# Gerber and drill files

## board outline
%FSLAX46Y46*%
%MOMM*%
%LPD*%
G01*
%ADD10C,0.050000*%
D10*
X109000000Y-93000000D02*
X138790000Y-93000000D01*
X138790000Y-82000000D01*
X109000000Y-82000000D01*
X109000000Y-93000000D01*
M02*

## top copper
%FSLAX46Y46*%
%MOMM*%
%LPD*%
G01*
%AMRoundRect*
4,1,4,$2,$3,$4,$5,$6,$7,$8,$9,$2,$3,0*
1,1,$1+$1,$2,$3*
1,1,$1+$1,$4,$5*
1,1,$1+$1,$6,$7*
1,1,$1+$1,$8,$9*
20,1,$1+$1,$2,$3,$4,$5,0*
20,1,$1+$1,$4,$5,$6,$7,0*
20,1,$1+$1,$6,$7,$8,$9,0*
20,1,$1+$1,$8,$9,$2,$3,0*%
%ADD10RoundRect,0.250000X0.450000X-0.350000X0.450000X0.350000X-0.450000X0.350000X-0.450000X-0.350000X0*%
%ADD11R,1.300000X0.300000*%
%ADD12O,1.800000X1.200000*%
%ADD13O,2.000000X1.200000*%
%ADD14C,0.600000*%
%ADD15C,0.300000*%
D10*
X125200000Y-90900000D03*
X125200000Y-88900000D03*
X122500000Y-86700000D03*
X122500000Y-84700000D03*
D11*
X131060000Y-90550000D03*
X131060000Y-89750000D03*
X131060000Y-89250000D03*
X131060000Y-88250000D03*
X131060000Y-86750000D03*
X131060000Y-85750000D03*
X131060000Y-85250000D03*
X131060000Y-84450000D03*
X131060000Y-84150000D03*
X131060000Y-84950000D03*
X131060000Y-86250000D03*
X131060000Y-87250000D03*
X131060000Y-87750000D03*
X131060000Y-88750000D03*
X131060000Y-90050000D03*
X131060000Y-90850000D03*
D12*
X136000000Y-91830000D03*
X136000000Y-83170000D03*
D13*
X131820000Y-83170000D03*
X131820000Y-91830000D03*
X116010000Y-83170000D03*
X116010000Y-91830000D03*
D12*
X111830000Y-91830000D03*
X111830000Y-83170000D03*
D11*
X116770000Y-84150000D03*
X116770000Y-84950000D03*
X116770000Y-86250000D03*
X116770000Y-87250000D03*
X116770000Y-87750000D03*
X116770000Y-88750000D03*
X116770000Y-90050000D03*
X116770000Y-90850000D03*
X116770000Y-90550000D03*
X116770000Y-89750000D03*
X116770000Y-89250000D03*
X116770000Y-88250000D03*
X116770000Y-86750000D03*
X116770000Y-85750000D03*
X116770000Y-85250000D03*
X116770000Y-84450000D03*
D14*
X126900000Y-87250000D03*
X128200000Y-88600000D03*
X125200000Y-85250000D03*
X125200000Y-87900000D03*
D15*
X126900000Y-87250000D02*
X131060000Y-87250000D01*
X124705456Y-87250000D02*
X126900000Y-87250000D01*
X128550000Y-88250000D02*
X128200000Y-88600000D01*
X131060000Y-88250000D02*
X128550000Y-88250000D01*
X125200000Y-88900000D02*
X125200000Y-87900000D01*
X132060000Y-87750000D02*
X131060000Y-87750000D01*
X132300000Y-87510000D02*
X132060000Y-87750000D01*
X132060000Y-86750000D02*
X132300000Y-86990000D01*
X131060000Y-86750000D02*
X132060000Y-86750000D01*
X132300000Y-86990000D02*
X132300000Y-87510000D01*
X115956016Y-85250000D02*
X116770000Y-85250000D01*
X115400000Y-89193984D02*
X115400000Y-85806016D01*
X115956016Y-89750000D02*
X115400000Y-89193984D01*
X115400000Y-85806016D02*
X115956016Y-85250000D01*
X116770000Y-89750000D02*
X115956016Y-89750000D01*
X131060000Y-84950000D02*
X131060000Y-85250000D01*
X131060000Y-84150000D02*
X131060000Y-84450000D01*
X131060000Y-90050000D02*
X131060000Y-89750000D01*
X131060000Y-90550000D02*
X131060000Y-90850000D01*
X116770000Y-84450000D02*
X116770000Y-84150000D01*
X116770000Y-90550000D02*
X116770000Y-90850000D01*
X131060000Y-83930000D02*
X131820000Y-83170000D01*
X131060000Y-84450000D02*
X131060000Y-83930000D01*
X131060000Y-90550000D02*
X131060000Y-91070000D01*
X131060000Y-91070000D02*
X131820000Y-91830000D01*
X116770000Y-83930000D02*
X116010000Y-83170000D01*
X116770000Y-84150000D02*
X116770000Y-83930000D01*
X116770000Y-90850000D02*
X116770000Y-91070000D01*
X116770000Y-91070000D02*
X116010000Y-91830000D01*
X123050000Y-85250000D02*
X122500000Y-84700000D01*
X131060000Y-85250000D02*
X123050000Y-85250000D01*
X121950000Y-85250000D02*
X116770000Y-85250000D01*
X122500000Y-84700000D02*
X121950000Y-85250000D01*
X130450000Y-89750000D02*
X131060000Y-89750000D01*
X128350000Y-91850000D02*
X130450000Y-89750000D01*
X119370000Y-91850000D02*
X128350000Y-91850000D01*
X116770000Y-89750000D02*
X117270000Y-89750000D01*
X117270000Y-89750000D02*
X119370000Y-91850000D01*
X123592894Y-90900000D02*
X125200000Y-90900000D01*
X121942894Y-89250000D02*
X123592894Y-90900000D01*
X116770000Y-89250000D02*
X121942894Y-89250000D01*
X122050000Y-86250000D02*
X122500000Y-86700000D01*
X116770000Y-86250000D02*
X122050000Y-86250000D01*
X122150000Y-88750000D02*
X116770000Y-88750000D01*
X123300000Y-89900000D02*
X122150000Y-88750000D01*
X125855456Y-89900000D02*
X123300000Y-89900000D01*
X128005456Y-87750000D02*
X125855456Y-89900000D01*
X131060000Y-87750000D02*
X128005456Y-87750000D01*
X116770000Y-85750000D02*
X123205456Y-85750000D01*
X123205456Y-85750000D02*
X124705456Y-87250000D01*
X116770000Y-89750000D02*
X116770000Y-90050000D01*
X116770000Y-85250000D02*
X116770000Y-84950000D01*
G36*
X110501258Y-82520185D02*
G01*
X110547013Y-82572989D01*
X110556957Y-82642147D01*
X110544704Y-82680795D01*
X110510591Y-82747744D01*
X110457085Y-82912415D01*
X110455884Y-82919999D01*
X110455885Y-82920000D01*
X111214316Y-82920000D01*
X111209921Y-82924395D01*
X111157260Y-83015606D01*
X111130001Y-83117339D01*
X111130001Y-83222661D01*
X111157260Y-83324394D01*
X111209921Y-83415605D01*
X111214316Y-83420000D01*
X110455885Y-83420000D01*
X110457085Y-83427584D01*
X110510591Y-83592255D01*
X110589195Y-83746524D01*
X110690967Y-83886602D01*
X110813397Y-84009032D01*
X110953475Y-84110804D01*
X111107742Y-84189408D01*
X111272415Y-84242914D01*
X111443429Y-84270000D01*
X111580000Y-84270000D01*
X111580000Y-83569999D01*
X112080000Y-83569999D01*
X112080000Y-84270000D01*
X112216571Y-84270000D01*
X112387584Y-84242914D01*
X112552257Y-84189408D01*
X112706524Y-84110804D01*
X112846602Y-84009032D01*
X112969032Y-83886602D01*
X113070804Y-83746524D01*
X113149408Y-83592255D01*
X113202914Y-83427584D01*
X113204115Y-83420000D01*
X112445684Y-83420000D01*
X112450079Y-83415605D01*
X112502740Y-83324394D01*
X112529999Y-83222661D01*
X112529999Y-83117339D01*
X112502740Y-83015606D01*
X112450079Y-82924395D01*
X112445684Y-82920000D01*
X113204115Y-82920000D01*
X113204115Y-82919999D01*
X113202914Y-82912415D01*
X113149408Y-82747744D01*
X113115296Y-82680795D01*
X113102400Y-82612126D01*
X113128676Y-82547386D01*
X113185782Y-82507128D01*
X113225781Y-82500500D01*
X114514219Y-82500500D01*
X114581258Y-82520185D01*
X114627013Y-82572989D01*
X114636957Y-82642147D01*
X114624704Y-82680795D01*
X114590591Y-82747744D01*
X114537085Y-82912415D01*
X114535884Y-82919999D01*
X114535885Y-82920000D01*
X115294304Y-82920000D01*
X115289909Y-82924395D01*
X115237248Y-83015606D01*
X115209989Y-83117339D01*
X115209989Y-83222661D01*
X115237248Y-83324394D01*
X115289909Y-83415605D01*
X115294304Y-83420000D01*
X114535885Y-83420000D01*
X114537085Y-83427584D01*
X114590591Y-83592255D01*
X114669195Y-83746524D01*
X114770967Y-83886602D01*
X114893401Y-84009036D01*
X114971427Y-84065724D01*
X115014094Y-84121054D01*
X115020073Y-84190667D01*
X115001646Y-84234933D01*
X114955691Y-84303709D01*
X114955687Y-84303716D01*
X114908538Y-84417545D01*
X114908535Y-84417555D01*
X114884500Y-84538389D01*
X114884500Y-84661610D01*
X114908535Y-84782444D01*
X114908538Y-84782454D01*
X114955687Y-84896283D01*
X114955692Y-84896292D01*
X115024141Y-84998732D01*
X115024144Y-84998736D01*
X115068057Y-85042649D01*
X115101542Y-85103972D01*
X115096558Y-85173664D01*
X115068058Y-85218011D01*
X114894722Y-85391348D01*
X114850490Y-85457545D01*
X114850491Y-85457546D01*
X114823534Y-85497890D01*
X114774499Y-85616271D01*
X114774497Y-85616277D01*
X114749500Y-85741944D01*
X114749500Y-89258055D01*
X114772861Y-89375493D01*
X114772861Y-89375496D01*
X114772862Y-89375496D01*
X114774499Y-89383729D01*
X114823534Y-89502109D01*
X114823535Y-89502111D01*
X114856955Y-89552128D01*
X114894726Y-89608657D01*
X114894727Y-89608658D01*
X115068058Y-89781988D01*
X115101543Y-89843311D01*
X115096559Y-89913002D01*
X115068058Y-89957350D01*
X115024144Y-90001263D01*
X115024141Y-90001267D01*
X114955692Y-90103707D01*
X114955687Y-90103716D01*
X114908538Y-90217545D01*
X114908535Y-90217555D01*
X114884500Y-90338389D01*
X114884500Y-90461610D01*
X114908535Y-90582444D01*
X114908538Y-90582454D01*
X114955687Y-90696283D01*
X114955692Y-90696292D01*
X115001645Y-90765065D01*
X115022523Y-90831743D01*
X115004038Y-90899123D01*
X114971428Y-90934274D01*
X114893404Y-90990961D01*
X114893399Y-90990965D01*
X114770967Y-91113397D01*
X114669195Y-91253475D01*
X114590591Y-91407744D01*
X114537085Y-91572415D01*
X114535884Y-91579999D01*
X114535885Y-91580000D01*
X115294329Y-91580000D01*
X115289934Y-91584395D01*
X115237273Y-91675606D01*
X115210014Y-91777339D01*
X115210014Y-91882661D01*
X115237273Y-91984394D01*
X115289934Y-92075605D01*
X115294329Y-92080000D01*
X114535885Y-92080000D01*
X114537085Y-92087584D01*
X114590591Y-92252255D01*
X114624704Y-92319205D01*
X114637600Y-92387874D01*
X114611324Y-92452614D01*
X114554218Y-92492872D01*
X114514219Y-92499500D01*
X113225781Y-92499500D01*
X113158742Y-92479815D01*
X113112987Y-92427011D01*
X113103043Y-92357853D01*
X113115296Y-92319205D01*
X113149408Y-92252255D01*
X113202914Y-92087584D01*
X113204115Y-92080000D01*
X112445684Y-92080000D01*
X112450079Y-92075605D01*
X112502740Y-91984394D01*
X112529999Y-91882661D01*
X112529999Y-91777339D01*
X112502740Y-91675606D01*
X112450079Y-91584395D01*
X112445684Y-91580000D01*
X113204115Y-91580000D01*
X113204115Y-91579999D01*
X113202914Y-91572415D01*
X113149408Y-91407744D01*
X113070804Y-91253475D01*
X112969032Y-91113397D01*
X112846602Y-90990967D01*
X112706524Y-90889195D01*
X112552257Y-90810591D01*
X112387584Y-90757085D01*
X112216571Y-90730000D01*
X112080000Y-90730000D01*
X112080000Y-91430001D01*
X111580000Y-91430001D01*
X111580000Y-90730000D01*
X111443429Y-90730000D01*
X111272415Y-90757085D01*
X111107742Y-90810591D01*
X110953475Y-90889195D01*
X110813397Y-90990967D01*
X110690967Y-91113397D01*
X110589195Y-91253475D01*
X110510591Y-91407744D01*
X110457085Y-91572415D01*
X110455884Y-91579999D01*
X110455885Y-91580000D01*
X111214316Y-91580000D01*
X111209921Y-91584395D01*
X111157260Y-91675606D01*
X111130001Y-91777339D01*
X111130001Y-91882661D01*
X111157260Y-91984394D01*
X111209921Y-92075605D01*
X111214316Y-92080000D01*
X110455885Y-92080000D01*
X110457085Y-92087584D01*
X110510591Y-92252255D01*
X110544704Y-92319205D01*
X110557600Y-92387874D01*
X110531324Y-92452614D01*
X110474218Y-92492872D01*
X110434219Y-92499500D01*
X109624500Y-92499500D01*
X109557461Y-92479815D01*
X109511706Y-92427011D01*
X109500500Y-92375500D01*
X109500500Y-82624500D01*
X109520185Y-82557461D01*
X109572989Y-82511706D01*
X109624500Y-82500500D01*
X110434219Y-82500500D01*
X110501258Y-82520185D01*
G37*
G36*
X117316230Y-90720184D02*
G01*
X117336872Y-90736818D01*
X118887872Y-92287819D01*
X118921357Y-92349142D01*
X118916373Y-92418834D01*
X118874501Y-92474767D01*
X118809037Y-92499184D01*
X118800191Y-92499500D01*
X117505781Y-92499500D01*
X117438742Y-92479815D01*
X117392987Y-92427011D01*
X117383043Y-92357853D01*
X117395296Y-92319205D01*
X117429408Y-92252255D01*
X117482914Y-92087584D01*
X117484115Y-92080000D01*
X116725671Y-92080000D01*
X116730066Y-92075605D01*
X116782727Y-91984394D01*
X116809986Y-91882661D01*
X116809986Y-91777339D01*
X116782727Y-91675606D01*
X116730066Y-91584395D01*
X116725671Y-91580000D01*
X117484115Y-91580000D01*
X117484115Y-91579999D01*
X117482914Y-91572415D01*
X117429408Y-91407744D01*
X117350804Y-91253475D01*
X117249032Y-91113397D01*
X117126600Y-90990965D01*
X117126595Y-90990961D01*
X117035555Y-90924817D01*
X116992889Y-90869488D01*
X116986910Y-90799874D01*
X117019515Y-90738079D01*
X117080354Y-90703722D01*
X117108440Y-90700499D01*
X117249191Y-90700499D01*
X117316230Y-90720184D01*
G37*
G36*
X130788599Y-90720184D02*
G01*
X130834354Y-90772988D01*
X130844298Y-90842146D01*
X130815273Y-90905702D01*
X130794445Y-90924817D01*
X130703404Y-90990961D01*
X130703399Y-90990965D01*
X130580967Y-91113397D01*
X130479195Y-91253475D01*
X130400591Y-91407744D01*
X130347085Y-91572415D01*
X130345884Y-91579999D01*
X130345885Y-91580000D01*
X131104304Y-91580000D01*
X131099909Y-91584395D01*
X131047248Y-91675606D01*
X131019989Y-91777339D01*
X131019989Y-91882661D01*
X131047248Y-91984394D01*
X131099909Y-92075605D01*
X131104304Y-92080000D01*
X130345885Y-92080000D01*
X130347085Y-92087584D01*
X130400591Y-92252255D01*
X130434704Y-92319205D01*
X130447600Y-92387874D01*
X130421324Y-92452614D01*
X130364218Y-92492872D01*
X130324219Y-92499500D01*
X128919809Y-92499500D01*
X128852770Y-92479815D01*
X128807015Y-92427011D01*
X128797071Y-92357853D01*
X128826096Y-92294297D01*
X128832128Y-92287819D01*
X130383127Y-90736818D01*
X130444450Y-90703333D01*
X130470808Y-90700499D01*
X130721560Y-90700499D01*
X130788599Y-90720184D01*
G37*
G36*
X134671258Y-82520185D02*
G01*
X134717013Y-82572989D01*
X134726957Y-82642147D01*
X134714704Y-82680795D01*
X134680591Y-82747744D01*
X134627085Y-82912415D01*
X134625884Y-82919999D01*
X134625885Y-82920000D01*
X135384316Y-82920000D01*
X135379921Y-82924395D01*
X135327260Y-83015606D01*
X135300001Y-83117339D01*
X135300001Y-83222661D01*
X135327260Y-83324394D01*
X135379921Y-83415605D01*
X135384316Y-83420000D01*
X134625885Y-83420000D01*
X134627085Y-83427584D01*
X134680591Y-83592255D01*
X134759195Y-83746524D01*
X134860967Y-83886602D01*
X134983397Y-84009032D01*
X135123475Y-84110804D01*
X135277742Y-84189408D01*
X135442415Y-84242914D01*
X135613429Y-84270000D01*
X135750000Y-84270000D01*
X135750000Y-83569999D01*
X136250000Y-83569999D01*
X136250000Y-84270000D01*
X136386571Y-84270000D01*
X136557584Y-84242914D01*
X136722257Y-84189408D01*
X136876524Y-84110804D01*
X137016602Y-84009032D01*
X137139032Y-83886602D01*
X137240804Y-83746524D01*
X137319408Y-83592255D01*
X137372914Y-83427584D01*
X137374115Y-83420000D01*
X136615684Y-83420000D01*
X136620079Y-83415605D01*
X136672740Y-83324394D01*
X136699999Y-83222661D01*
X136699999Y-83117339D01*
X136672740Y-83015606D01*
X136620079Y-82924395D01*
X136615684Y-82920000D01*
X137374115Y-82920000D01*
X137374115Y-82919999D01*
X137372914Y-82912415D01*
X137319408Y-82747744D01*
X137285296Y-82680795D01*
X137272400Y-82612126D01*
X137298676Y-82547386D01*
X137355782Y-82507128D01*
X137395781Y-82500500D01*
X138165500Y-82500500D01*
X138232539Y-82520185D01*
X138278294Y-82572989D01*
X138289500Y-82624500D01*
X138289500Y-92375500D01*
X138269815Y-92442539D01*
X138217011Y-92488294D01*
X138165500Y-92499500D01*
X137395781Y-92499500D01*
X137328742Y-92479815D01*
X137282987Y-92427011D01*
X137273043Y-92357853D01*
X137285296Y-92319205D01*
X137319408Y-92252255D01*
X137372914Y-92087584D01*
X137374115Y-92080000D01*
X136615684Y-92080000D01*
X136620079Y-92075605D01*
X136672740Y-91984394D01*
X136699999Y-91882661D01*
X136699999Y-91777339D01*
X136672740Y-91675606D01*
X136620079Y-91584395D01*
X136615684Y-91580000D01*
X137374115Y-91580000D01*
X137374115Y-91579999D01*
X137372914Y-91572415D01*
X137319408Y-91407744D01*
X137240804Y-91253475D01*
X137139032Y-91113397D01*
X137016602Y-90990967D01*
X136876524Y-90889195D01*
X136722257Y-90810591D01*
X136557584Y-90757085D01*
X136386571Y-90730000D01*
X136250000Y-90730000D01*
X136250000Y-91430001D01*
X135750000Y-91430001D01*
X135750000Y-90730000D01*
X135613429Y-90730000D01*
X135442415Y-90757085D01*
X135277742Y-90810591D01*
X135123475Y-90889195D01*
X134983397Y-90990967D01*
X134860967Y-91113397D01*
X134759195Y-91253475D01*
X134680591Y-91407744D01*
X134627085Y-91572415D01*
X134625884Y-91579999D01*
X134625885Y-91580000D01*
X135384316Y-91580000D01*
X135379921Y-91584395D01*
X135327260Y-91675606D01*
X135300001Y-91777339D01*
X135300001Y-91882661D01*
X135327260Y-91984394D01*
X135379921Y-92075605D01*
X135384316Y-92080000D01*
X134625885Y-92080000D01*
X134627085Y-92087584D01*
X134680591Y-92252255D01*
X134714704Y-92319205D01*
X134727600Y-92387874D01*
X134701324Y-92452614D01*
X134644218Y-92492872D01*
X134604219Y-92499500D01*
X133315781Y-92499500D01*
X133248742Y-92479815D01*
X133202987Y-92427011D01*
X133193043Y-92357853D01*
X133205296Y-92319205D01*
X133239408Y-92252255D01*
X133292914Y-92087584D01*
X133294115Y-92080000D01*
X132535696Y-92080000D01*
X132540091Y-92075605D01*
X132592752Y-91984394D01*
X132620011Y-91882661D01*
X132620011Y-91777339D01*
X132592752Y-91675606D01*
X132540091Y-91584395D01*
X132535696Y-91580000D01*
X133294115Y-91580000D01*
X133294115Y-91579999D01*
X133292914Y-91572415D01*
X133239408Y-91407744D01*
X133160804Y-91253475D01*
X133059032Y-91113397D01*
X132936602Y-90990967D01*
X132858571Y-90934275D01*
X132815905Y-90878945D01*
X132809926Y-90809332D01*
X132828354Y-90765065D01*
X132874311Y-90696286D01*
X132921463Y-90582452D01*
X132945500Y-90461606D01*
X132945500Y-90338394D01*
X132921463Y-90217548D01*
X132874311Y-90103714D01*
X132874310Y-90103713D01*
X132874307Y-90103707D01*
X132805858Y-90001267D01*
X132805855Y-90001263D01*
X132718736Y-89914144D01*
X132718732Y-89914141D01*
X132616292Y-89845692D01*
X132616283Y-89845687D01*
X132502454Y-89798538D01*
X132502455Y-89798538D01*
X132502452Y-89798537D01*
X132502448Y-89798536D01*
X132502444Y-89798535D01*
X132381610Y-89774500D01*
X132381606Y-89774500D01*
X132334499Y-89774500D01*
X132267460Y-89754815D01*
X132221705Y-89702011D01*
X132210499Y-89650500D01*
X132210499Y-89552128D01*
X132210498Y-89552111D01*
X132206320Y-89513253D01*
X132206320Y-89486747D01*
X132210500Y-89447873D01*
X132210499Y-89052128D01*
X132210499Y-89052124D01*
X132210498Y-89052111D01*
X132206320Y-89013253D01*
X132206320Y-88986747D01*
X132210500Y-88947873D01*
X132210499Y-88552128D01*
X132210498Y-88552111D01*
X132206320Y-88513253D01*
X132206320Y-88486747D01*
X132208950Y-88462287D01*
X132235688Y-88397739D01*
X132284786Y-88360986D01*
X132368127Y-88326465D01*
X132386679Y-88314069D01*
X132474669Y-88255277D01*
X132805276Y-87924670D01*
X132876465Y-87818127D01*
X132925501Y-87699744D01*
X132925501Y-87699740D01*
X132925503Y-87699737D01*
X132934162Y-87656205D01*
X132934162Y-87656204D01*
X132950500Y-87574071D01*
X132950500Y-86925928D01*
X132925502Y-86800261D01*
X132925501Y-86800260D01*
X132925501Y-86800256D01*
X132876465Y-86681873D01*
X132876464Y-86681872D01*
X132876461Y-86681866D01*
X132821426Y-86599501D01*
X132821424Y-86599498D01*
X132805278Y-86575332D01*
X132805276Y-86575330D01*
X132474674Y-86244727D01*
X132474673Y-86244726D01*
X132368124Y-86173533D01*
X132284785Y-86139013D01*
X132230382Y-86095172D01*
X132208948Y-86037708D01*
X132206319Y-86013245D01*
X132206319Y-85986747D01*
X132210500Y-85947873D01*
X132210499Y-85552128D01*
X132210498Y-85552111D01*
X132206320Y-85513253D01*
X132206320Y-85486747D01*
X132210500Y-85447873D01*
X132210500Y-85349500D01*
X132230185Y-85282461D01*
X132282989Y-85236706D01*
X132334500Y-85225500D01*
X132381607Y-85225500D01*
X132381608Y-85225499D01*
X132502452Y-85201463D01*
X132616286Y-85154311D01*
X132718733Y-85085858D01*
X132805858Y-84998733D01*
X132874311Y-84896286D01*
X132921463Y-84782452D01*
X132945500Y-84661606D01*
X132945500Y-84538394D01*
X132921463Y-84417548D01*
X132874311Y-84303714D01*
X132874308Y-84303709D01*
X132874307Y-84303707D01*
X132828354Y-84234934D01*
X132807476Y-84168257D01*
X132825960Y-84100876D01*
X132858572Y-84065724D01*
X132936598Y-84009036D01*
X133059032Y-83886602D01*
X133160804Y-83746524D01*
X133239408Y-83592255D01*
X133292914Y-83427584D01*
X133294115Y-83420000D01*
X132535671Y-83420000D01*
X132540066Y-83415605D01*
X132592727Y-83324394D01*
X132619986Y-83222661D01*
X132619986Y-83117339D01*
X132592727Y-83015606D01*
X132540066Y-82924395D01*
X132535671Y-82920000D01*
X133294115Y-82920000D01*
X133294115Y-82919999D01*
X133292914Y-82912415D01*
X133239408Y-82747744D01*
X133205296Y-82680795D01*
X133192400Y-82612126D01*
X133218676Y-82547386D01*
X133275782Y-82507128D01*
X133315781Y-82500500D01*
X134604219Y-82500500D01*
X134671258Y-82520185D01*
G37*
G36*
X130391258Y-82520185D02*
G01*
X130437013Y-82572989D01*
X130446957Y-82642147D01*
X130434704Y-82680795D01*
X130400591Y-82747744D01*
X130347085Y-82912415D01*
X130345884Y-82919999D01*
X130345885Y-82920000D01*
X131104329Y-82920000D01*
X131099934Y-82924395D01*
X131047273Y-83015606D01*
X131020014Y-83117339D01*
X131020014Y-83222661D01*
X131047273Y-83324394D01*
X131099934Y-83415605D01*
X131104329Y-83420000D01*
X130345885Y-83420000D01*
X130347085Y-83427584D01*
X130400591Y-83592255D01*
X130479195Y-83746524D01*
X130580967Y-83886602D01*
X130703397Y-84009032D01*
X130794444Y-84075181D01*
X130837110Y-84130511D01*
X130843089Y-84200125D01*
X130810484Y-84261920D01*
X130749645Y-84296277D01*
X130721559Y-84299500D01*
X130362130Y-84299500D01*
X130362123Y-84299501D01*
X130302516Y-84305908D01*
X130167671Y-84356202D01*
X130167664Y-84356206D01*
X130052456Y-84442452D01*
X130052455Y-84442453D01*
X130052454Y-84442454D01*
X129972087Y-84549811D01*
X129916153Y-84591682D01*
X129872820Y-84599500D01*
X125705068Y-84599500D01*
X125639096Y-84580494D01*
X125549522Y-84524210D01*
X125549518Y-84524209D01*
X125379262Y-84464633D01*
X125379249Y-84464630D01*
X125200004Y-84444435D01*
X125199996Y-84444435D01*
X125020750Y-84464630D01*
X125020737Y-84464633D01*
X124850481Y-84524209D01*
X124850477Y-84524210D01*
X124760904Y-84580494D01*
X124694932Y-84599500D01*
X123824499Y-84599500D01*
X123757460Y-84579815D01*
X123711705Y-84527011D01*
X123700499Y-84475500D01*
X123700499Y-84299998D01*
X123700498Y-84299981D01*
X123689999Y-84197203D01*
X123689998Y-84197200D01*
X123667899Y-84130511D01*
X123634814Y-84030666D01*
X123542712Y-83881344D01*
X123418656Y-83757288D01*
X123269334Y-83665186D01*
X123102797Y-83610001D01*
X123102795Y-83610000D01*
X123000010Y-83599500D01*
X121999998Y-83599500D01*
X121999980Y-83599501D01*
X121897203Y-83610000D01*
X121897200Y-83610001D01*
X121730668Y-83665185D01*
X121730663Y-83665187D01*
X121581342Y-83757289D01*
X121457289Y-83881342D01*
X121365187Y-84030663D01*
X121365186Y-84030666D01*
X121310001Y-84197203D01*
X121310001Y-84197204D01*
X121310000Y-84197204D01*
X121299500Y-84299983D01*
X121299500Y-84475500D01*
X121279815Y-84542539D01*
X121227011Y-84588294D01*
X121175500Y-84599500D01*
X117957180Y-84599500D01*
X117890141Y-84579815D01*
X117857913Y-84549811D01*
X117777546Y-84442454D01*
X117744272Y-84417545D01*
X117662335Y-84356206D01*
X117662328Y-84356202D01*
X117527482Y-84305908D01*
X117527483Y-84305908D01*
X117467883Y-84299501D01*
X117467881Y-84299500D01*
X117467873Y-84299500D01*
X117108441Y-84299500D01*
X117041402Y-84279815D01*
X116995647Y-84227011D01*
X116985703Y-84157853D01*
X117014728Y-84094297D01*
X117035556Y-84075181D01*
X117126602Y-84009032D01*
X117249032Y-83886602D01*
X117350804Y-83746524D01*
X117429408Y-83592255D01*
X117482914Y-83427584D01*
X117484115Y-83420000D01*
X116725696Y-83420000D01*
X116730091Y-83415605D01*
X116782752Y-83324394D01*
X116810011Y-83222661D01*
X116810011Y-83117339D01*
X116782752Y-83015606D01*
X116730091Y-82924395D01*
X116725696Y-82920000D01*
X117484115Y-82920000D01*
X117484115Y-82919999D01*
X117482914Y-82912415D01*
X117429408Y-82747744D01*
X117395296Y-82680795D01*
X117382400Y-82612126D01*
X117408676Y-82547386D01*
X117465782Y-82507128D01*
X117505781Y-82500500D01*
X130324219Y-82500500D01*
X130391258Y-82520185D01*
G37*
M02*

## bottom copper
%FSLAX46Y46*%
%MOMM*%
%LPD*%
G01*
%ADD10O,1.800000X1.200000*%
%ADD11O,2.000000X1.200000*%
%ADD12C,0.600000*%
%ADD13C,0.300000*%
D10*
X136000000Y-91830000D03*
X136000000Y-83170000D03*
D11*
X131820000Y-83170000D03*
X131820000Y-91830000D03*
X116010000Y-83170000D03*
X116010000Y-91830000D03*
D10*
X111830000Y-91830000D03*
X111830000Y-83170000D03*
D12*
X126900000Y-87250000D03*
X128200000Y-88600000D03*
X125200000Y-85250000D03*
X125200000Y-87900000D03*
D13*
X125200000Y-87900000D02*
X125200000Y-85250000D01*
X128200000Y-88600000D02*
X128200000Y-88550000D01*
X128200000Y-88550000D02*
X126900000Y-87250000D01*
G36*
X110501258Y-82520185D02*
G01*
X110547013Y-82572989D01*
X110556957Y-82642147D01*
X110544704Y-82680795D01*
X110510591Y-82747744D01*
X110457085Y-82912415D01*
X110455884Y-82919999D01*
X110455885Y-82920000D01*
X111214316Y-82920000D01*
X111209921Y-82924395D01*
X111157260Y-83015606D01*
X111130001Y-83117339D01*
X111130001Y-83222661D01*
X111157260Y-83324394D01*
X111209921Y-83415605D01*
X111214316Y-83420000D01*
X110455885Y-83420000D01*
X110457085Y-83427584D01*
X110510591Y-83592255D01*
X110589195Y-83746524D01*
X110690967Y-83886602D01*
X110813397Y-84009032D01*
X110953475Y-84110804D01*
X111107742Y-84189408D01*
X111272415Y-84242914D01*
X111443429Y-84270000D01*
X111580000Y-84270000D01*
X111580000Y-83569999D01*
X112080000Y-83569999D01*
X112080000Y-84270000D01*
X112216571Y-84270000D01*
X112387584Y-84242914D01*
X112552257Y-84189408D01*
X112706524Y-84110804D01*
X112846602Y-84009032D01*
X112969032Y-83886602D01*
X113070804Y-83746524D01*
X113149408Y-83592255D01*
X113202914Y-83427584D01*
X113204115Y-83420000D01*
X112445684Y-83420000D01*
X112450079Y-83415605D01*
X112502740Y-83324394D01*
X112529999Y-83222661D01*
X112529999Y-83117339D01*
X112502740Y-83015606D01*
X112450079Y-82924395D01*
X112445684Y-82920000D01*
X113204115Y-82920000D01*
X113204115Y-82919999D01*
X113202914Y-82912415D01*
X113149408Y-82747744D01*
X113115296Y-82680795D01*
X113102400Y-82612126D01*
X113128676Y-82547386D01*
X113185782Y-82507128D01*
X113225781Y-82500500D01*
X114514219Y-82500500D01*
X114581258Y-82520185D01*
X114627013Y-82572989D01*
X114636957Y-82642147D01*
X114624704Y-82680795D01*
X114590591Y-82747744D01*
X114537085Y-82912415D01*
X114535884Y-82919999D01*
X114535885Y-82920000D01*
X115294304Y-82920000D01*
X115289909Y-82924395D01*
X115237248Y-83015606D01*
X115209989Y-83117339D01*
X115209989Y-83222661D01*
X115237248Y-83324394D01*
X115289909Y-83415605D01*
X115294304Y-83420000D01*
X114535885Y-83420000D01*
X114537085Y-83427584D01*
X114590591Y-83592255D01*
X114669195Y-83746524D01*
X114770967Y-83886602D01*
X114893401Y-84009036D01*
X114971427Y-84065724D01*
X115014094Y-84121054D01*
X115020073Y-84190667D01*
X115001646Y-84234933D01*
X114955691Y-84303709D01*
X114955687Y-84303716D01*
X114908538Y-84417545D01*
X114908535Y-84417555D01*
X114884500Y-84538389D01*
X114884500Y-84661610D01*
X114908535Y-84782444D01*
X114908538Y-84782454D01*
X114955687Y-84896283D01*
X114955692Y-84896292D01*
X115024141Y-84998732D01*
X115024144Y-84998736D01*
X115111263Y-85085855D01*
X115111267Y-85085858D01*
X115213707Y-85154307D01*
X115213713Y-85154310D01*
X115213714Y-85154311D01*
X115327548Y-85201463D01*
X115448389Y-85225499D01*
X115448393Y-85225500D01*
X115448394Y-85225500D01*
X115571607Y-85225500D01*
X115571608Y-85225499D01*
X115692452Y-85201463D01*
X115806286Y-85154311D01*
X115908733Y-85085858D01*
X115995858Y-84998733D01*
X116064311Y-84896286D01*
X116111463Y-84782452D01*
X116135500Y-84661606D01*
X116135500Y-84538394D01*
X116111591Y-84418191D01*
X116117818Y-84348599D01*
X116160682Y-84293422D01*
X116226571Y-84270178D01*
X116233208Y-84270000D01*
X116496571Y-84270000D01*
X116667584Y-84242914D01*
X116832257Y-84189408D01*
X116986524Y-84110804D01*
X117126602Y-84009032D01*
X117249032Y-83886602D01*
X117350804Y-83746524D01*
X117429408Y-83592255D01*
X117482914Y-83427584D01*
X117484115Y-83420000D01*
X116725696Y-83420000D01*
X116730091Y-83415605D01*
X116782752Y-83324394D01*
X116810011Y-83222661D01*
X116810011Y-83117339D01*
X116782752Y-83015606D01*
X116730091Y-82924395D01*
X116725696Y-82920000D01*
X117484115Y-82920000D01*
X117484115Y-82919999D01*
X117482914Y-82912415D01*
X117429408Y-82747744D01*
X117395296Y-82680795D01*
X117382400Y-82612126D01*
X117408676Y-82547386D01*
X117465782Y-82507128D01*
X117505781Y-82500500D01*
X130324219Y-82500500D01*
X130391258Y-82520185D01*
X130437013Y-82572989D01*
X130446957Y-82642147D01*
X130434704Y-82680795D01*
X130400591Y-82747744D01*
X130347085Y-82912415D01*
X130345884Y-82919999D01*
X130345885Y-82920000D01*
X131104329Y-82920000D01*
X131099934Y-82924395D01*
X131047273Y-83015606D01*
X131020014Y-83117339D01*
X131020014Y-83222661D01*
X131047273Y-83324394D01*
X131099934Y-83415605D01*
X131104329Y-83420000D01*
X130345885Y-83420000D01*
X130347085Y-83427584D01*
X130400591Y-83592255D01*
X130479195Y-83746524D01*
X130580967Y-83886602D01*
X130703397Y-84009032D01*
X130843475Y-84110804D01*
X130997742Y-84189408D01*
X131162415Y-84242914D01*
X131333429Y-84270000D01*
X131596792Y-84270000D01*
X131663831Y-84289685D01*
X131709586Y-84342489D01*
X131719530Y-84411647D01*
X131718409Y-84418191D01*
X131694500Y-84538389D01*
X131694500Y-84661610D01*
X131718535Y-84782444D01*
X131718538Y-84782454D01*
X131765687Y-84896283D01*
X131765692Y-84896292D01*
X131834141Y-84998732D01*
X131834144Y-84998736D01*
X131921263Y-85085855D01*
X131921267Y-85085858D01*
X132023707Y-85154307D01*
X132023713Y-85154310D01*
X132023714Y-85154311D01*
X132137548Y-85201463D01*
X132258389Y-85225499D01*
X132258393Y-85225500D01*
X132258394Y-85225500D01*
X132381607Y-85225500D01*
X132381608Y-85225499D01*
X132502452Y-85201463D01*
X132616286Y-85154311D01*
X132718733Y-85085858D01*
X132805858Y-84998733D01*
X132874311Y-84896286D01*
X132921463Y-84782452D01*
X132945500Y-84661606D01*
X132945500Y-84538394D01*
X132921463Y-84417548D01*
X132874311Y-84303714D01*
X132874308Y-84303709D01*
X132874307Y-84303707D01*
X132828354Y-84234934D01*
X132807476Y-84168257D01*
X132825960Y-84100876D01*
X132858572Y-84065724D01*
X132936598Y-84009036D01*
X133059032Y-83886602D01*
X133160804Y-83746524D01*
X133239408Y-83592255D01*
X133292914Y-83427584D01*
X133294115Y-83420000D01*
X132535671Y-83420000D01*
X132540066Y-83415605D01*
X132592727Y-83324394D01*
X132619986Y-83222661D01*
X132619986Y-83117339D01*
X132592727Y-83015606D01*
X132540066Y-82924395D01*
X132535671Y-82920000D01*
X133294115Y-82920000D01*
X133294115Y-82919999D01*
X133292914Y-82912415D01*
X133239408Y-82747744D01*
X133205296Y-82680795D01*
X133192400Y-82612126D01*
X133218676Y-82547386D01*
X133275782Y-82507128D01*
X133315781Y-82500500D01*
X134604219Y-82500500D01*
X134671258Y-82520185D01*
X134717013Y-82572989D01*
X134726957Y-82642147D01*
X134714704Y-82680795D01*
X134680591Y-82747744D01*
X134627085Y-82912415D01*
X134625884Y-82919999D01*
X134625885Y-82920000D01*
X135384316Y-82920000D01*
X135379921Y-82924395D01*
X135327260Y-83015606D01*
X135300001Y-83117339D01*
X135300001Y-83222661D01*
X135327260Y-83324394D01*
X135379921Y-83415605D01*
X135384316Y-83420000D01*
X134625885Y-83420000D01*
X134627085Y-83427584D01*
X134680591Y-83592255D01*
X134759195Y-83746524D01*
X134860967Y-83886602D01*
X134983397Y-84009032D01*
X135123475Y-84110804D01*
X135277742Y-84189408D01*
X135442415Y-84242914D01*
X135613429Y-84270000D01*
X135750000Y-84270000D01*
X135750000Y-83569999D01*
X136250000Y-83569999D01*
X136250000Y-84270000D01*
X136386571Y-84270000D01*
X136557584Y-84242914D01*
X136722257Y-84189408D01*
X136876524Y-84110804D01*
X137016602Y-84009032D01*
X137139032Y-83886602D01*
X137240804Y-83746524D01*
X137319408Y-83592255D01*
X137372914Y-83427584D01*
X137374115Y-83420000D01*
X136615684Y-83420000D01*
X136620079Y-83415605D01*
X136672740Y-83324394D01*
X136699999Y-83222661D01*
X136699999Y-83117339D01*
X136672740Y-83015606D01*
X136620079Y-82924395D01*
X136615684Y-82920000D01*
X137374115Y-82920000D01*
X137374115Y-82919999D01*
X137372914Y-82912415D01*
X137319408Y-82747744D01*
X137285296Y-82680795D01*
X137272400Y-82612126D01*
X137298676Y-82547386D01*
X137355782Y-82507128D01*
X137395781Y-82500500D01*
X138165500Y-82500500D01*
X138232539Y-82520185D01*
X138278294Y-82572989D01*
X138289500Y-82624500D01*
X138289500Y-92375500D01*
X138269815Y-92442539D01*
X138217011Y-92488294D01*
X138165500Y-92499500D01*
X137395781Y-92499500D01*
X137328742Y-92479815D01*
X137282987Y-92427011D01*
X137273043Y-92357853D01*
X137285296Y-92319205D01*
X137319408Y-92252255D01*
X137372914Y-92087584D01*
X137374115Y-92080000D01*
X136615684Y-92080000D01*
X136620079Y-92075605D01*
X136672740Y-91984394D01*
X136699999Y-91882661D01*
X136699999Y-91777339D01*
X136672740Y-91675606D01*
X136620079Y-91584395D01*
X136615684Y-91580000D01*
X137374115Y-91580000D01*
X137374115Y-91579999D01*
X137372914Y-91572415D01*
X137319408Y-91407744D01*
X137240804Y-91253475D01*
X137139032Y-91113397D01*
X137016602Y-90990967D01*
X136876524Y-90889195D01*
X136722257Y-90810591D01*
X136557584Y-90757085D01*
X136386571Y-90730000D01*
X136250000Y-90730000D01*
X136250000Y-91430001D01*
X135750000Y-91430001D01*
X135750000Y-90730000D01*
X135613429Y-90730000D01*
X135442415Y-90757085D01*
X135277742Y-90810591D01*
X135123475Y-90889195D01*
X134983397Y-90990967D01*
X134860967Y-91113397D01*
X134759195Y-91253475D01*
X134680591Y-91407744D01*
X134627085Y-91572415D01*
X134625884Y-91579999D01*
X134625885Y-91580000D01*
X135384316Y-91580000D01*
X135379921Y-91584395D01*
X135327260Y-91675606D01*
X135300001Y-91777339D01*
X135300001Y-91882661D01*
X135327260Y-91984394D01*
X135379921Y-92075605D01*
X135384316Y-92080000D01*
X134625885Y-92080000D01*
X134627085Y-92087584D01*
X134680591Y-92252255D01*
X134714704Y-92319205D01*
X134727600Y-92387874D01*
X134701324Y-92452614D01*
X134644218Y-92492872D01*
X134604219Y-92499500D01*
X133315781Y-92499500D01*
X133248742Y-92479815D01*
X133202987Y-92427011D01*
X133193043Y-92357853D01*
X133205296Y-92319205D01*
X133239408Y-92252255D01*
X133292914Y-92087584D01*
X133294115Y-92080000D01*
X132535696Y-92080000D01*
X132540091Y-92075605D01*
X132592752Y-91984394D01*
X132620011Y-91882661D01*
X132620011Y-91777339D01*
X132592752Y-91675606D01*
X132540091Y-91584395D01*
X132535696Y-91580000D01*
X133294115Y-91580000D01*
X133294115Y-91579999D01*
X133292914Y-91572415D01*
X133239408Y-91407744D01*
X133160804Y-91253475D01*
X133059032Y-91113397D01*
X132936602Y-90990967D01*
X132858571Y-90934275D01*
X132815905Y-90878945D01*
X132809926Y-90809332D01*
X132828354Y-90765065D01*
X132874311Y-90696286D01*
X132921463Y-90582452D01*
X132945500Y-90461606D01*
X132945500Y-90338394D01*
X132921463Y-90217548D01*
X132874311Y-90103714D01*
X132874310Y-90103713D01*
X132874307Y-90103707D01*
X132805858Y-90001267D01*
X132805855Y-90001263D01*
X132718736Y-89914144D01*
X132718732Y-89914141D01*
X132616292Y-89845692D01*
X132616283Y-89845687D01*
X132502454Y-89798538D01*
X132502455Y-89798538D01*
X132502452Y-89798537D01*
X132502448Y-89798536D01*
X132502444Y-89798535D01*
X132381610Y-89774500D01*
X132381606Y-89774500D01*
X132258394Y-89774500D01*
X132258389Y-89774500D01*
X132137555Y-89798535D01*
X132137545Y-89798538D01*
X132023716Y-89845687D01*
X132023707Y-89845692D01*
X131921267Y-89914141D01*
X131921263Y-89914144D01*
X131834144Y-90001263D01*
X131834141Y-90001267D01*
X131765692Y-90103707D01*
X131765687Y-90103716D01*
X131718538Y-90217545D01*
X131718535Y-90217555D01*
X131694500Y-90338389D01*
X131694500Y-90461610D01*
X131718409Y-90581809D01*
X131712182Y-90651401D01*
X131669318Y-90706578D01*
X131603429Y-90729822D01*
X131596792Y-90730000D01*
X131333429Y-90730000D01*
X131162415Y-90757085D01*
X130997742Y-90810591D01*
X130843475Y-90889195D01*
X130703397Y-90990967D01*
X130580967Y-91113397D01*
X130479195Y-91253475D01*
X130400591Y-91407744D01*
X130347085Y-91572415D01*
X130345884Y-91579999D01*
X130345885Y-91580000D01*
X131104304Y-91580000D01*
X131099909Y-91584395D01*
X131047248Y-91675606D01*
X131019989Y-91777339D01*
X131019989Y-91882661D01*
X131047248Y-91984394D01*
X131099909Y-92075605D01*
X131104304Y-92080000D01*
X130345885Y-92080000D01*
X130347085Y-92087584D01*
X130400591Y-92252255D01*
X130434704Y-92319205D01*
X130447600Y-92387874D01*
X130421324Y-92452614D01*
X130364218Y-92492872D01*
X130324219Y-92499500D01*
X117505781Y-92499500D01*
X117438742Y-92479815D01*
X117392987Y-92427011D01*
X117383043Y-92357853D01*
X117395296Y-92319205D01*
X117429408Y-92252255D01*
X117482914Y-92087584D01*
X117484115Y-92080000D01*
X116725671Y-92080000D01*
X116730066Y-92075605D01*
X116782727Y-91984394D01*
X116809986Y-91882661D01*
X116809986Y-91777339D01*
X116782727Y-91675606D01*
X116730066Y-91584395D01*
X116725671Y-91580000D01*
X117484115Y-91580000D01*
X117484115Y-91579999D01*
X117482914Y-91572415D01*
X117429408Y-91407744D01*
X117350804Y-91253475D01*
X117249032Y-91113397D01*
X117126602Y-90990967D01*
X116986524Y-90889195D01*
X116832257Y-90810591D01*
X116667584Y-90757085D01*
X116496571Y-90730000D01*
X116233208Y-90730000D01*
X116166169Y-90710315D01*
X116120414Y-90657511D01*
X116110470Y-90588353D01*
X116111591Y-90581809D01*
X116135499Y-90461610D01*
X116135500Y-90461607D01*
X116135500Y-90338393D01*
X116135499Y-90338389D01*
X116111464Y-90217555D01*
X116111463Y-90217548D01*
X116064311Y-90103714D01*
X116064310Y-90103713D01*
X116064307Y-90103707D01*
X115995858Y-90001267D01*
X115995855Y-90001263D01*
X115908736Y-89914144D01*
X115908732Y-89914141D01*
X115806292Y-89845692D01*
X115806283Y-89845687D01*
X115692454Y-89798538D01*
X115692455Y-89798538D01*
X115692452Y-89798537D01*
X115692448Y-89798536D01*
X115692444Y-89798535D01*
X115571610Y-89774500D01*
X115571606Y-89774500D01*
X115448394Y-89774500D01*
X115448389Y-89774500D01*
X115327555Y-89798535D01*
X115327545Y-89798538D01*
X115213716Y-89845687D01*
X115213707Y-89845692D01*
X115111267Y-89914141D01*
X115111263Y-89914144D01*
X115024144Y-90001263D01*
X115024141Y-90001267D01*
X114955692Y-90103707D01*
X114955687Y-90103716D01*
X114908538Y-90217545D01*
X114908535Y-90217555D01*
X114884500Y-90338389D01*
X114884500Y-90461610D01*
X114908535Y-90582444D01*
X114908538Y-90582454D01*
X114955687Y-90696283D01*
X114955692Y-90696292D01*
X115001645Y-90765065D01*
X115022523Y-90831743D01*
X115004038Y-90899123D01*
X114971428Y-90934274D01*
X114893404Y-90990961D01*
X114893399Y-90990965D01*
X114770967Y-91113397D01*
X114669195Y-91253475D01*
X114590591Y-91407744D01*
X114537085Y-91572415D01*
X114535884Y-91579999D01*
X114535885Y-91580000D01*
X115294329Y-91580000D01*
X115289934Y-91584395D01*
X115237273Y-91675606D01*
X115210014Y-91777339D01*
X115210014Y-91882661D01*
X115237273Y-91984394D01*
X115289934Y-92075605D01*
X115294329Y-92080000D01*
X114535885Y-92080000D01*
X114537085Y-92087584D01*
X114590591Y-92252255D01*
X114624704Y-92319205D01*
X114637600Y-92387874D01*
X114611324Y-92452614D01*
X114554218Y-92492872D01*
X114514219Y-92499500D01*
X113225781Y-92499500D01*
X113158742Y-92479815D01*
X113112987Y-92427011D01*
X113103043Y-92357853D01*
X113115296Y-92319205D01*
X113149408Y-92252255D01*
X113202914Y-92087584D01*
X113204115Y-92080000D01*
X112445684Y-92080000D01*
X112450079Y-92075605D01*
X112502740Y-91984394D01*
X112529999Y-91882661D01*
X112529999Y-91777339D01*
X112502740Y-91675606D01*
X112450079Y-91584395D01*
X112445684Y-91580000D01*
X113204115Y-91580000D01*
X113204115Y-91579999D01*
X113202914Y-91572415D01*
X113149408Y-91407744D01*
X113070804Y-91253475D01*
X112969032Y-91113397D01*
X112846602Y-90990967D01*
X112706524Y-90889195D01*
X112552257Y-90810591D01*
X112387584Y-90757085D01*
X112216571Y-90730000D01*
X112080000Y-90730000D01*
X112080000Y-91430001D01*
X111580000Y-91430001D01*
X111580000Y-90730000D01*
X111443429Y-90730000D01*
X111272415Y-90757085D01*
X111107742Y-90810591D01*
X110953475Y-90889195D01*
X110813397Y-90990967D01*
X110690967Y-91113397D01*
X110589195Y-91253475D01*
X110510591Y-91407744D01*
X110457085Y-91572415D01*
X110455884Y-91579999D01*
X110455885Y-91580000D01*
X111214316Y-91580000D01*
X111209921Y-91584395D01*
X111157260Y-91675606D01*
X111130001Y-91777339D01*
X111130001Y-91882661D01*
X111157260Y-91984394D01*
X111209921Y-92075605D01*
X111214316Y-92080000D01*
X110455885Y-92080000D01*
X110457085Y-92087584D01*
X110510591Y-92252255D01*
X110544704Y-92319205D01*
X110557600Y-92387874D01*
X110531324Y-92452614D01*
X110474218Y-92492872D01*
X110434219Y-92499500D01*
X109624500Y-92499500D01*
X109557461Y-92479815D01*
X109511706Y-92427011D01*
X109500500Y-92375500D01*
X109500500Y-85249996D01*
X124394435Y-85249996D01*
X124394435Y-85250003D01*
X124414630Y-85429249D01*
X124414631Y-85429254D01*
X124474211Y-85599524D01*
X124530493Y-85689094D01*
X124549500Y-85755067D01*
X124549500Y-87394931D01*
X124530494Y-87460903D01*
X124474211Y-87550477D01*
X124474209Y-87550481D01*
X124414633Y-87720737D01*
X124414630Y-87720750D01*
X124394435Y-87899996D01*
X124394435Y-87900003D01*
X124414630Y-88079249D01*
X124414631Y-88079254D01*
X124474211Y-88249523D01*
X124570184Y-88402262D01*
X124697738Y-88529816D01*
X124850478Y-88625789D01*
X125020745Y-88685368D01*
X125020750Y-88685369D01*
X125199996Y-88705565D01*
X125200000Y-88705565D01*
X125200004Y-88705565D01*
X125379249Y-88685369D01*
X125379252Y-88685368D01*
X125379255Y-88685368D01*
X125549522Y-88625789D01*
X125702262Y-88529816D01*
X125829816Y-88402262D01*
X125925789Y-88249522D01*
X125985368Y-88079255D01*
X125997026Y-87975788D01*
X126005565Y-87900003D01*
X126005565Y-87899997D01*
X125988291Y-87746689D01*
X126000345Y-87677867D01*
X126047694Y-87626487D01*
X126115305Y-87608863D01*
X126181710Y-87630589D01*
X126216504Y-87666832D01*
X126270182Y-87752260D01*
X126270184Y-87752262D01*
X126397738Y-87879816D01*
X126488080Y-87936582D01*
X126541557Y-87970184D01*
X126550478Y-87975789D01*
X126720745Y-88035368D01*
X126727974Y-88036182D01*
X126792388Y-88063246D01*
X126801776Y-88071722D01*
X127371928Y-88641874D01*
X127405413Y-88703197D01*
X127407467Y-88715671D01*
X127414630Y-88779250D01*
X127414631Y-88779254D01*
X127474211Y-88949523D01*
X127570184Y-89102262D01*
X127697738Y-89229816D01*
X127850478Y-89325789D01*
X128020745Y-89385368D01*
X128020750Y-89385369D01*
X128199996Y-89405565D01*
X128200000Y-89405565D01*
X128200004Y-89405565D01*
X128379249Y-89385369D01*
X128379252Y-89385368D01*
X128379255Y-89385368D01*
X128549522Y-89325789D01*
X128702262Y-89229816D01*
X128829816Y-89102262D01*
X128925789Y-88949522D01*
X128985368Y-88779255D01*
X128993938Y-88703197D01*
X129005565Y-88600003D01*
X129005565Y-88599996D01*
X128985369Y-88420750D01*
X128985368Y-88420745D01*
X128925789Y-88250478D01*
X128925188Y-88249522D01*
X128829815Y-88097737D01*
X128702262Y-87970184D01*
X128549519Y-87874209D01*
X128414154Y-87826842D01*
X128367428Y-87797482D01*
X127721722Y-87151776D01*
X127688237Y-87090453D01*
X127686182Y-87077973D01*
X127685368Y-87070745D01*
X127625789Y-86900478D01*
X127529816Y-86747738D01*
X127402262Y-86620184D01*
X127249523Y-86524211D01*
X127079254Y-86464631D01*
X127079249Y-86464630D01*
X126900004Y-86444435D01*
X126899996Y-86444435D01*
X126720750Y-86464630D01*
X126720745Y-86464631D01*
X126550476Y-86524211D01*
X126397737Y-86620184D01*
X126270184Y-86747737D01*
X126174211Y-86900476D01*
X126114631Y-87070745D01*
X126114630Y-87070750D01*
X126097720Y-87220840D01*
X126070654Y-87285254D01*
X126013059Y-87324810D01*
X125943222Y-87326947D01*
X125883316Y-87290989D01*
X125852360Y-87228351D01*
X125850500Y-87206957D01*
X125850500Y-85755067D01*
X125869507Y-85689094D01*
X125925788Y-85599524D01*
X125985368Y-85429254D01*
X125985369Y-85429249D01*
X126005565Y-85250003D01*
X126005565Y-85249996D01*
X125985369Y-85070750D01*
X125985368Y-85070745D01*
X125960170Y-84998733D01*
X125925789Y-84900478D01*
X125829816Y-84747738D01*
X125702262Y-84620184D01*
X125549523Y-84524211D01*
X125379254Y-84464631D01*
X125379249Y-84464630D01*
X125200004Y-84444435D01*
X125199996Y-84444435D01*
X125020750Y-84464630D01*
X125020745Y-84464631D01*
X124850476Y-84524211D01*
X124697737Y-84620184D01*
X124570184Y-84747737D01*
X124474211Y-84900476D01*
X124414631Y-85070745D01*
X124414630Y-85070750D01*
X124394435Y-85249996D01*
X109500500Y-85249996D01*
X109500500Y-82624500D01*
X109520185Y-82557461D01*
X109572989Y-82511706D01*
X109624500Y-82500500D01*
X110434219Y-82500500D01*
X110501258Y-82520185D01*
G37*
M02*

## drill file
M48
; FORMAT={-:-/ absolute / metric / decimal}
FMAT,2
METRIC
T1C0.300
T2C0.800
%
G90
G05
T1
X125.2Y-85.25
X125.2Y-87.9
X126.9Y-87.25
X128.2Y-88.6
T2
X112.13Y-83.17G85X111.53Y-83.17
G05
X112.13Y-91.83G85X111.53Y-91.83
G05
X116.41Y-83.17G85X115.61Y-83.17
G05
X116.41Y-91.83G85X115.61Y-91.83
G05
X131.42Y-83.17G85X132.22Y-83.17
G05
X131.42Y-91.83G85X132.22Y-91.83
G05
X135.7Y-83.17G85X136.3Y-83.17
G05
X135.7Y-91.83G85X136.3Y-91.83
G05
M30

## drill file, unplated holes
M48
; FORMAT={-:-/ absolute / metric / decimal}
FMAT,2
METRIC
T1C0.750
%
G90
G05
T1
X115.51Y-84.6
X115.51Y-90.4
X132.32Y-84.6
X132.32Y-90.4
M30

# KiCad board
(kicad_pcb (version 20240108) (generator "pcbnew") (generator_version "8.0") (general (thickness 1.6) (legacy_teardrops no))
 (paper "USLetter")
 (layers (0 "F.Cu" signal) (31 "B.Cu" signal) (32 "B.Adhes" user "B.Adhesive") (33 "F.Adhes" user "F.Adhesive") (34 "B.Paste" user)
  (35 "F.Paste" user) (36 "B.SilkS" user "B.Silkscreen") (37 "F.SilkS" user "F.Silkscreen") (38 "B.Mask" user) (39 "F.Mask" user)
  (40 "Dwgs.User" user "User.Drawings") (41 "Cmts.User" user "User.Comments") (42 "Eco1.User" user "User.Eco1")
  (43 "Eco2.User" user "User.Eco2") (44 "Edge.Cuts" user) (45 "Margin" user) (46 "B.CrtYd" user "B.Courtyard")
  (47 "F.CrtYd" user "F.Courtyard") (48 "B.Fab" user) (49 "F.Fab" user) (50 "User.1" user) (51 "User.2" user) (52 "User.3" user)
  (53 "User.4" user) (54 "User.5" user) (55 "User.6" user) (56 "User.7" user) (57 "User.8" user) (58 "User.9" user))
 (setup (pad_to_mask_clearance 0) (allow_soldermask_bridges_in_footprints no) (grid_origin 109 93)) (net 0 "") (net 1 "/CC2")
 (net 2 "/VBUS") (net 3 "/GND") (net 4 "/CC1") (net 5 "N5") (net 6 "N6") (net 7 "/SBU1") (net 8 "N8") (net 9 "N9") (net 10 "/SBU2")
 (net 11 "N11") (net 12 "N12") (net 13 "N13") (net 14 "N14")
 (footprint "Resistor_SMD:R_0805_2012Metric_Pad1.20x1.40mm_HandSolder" (layer "F.Cu") (at 125.2 89.9 90)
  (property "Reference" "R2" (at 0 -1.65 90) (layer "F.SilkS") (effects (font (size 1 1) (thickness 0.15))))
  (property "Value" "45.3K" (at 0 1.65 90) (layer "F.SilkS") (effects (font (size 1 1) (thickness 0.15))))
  (pad "1" smd roundrect (at -1 0 90) (size 1.2 1.4) (layers "F.Cu" "F.Paste" "F.Mask") (roundrect_rratio 0.208333) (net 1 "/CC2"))
  (pad "2" smd roundrect (at 1 0 90) (size 1.2 1.4) (layers "F.Cu" "F.Paste" "F.Mask") (roundrect_rratio 0.208333) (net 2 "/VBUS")))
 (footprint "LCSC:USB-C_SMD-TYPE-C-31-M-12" (layer "F.Cu") (at 114.3 87.5 -90)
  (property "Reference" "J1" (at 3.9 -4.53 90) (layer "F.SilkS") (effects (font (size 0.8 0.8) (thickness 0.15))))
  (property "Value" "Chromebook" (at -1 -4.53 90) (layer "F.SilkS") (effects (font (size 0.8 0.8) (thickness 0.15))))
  (pad "" np_thru_hole circle (at -2.9 -1.21 270) (size 0.75 0.75) (drill 0.75) (layers "F&B.Cu" "*.Mask"))
  (pad "" np_thru_hole circle (at 2.9 -1.21 270) (size 0.75 0.75) (drill 0.75) (layers "F&B.Cu" "*.Mask"))
  (pad "0" thru_hole oval (at -4.33 -1.71 270) (size 1.2 2) (drill oval 0.799998 1.600022) (layers "*.Cu" "*.Mask")
   (remove_unused_layers no) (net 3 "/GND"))
  (pad "1" thru_hole oval (at 4.33 -1.71 270) (size 1.2 2) (drill oval 0.799998 1.599971) (layers "*.Cu" "*.Mask") (remove_unused_layers no)
   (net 3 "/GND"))
  (pad "2" thru_hole oval (at 4.33 2.47 270) (size 1.2 1.8) (drill oval 0.799998 1.399997) (layers "*.Cu" "*.Mask")
   (remove_unused_layers no) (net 3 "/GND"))
  (pad "3" thru_hole oval (at -4.33 2.47 270) (size 1.2 1.8) (drill oval 0.799998 1.399997) (layers "*.Cu" "*.Mask")
   (remove_unused_layers no) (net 3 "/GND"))
  (pad "A1" smd rect (at -3.35 -2.47 270) (size 0.3 1.3) (layers "F.Cu" "F.Paste" "F.Mask") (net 3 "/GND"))
  (pad "A4" smd rect (at -2.55 -2.47 270) (size 0.3 1.3) (layers "F.Cu" "F.Paste" "F.Mask") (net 2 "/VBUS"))
  (pad "A5" smd rect (at -1.25 -2.47 270) (size 0.3 1.3) (layers "F.Cu" "F.Paste" "F.Mask") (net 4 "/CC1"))
  (pad "A6" smd rect (at -0.25 -2.47 270) (size 0.3 1.3) (layers "F.Cu" "F.Paste" "F.Mask") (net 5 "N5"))
  (pad "A7" smd rect (at 0.25 -2.47 270) (size 0.3 1.3) (layers "F.Cu" "F.Paste" "F.Mask") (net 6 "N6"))
  (pad "A8" smd rect (at 1.25 -2.47 270) (size 0.3 1.3) (layers "F.Cu" "F.Paste" "F.Mask") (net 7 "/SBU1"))
  (pad "A9" smd rect (at 2.55 -2.47 270) (size 0.3 1.3) (layers "F.Cu" "F.Paste" "F.Mask") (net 2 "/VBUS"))
  (pad "A12" smd rect (at 3.35 -2.47 270) (size 0.3 1.3) (layers "F.Cu" "F.Paste" "F.Mask") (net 3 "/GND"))
  (pad "B1" smd rect (at 3.05 -2.47 270) (size 0.3 1.3) (layers "F.Cu" "F.Paste" "F.Mask") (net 3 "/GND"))
  (pad "B4" smd rect (at 2.25 -2.47 270) (size 0.3 1.3) (layers "F.Cu" "F.Paste" "F.Mask") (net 2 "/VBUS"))
  (pad "B5" smd rect (at 1.75 -2.47 270) (size 0.3 1.3) (layers "F.Cu" "F.Paste" "F.Mask") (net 1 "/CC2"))
  (pad "B6" smd rect (at 0.75 -2.47 270) (size 0.3 1.3) (layers "F.Cu" "F.Paste" "F.Mask") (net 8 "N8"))
  (pad "B7" smd rect (at -0.75 -2.47 270) (size 0.3 1.3) (layers "F.Cu" "F.Paste" "F.Mask") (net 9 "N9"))
  (pad "B8" smd rect (at -1.75 -2.47 270) (size 0.3 1.3) (layers "F.Cu" "F.Paste" "F.Mask") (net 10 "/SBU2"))
  (pad "B9" smd rect (at -2.25 -2.47 270) (size 0.3 1.3) (layers "F.Cu" "F.Paste" "F.Mask") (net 2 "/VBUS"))
  (pad "B12" smd rect (at -3.05 -2.47 270) (size 0.3 1.3) (layers "F.Cu" "F.Paste" "F.Mask") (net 3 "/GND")))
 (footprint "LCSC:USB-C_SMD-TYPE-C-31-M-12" (layer "F.Cu") (at 133.53 87.5 90)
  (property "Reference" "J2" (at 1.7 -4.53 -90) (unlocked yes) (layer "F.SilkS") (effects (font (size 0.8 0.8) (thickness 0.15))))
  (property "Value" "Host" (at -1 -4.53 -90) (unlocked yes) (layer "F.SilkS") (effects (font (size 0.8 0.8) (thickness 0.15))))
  (pad "" np_thru_hole circle (at -2.9 -1.21 90) (size 0.75 0.75) (drill 0.75) (layers "F&B.Cu" "*.Mask"))
  (pad "" np_thru_hole circle (at 2.9 -1.21 90) (size 0.75 0.75) (drill 0.75) (layers "F&B.Cu" "*.Mask"))
  (pad "0" thru_hole oval (at -4.33 -1.71 90) (size 1.2 2) (drill oval 0.799998 1.600022) (layers "*.Cu" "*.Mask") (remove_unused_layers no)
   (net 3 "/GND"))
  (pad "1" thru_hole oval (at 4.33 -1.71 90) (size 1.2 2) (drill oval 0.799998 1.599971) (layers "*.Cu" "*.Mask") (remove_unused_layers no)
   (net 3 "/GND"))
  (pad "2" thru_hole oval (at 4.33 2.47 90) (size 1.2 1.8) (drill oval 0.799998 1.399997) (layers "*.Cu" "*.Mask") (remove_unused_layers no)
   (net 3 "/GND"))
  (pad "3" thru_hole oval (at -4.33 2.47 90) (size 1.2 1.8) (drill oval 0.799998 1.399997) (layers "*.Cu" "*.Mask")
   (remove_unused_layers no) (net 3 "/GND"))
  (pad "A1" smd rect (at -3.35 -2.47 90) (size 0.3 1.3) (layers "F.Cu" "F.Paste" "F.Mask") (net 3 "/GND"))
  (pad "A4" smd rect (at -2.55 -2.47 90) (size 0.3 1.3) (layers "F.Cu" "F.Paste" "F.Mask") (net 2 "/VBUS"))
  (pad "A5" smd rect (at -1.25 -2.47 90) (size 0.3 1.3) (layers "F.Cu" "F.Paste" "F.Mask") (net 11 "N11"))
  (pad "A6" smd rect (at -0.25 -2.47 90) (size 0.3 1.3) (layers "F.Cu" "F.Paste" "F.Mask") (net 7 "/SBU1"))
  (pad "A7" smd rect (at 0.25 -2.47 90) (size 0.3 1.3) (layers "F.Cu" "F.Paste" "F.Mask") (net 10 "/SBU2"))
  (pad "A8" smd rect (at 1.25 -2.47 90) (size 0.3 1.3) (layers "F.Cu" "F.Paste" "F.Mask") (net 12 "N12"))
  (pad "A9" smd rect (at 2.55 -2.47 90) (size 0.3 1.3) (layers "F.Cu" "F.Paste" "F.Mask") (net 2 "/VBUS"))
  (pad "A12" smd rect (at 3.35 -2.47 90) (size 0.3 1.3) (layers "F.Cu" "F.Paste" "F.Mask") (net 3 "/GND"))
  (pad "B1" smd rect (at 3.05 -2.47 90) (size 0.3 1.3) (layers "F.Cu" "F.Paste" "F.Mask") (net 3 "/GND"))
  (pad "B4" smd rect (at 2.25 -2.47 90) (size 0.3 1.3) (layers "F.Cu" "F.Paste" "F.Mask") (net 2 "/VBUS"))
  (pad "B5" smd rect (at 1.75 -2.47 90) (size 0.3 1.3) (layers "F.Cu" "F.Paste" "F.Mask") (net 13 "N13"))
  (pad "B6" smd rect (at 0.75 -2.47 90) (size 0.3 1.3) (layers "F.Cu" "F.Paste" "F.Mask") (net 7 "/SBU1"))
  (pad "B7" smd rect (at -0.75 -2.47 90) (size 0.3 1.3) (layers "F.Cu" "F.Paste" "F.Mask") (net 10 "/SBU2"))
  (pad "B8" smd rect (at -1.75 -2.47 90) (size 0.3 1.3) (layers "F.Cu" "F.Paste" "F.Mask") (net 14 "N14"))
  (pad "B9" smd rect (at -2.25 -2.47 90) (size 0.3 1.3) (layers "F.Cu" "F.Paste" "F.Mask") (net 2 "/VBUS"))
  (pad "B12" smd rect (at -3.05 -2.47 90) (size 0.3 1.3) (layers "F.Cu" "F.Paste" "F.Mask") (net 3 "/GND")))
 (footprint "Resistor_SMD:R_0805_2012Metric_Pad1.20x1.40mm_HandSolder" (layer "F.Cu") (at 122.5 85.7 90)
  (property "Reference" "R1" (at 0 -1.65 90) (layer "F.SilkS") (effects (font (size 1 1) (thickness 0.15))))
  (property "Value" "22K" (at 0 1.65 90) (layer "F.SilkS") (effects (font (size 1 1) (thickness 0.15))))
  (pad "1" smd roundrect (at -1 0 90) (size 1.2 1.4) (layers "F.Cu" "F.Paste" "F.Mask") (roundrect_rratio 0.208333) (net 4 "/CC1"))
  (pad "2" smd roundrect (at 1 0 90) (size 1.2 1.4) (layers "F.Cu" "F.Paste" "F.Mask") (roundrect_rratio 0.208333) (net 2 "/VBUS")))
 (gr_rect (start 109 93) (end 138.79 82) (stroke (width 0.05) (type default)) (fill none) (layer "Edge.Cuts"))
 (segment (start 128.55 88.25) (end 128.2 88.6) (width 0.3) (layer "F.Cu") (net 10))
 (segment (start 126.9 87.25) (end 131.06 87.25) (width 0.3) (layer "F.Cu") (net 10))
 (segment (start 124.705456 87.25) (end 126.9 87.25) (width 0.3) (layer "F.Cu") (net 10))
 (segment (start 123.205456 85.75) (end 124.705456 87.25) (width 0.3) (layer "F.Cu") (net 10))
 (segment (start 131.06 88.25) (end 128.55 88.25) (width 0.3) (layer "F.Cu") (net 10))
 (segment (start 116.77 85.75) (end 123.205456 85.75) (width 0.3) (layer "F.Cu") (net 10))
 (via (at 128.2 88.6) (size 0.6) (drill 0.3) (layers "F.Cu" "B.Cu") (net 10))
 (via (at 126.9 87.25) (size 0.6) (drill 0.3) (layers "F.Cu" "B.Cu") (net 10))
 (segment (start 128.2 88.6) (end 128.2 88.55) (width 0.3) (layer "B.Cu") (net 10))
 (segment (start 128.2 88.55) (end 126.9 87.25) (width 0.3) (layer "B.Cu") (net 10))
 (segment (start 116.77 83.93) (end 116.01 83.17) (width 0.3) (layer "F.Cu") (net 3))
 (segment (start 116.77 90.85) (end 116.77 91.07) (width 0.3) (layer "F.Cu") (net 3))
 (segment (start 116.77 84.45) (end 116.77 84.15) (width 0.3) (layer "F.Cu") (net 3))
 (segment (start 131.06 91.07) (end 131.82 91.83) (width 0.3) (layer "F.Cu") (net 3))
 (segment (start 131.06 83.93) (end 131.82 83.17) (width 0.3) (layer "F.Cu") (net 3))
 (segment (start 116.77 90.55) (end 116.77 90.85) (width 0.3) (layer "F.Cu") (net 3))
 (segment (start 131.06 84.45) (end 131.06 83.93) (width 0.3) (layer "F.Cu") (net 3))
 (segment (start 131.06 90.55) (end 131.06 90.85) (width 0.3) (layer "F.Cu") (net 3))
 (segment (start 116.77 84.15) (end 116.77 83.93) (width 0.3) (layer "F.Cu") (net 3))
 (segment (start 131.06 90.55) (end 131.06 91.07) (width 0.3) (layer "F.Cu") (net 3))
 (segment (start 131.06 84.15) (end 131.06 84.45) (width 0.3) (layer "F.Cu") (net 3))
 (segment (start 116.77 91.07) (end 116.01 91.83) (width 0.3) (layer "F.Cu") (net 3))
 (segment (start 119.37 91.85) (end 128.35 91.85) (width 0.3) (layer "F.Cu") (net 2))
 (segment (start 116.77 89.75) (end 117.27 89.75) (width 0.3) (layer "F.Cu") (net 2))
 (segment (start 117.27 89.75) (end 119.37 91.85) (width 0.3) (layer "F.Cu") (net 2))
 (segment (start 125.2 88.9) (end 125.2 87.9) (width 0.3) (layer "F.Cu") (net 2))
 (segment (start 131.06 85.25) (end 123.05 85.25) (width 0.3) (layer "F.Cu") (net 2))
 (segment (start 121.95 85.25) (end 116.77 85.25) (width 0.3) (layer "F.Cu") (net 2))
 (segment (start 116.77 89.75) (end 116.77 90.05) (width 0.3) (layer "F.Cu") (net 2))
 (segment (start 122.5 84.7) (end 121.95 85.25) (width 0.3) (layer "F.Cu") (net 2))
 (segment (start 123.05 85.25) (end 122.5 84.7) (width 0.3) (layer "F.Cu") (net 2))
 (segment (start 115.4 89.193984) (end 115.4 85.806016) (width 0.3) (layer "F.Cu") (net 2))
 (segment (start 130.45 89.75) (end 131.06 89.75) (width 0.3) (layer "F.Cu") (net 2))
 (segment (start 115.4 85.806016) (end 115.956016 85.25) (width 0.3) (layer "F.Cu") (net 2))
 (segment (start 131.06 84.95) (end 131.06 85.25) (width 0.3) (layer "F.Cu") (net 2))
 (segment (start 116.77 89.75) (end 115.956016 89.75) (width 0.3) (layer "F.Cu") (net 2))
 (segment (start 115.956016 85.25) (end 116.77 85.25) (width 0.3) (layer "F.Cu") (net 2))
 (segment (start 131.06 90.05) (end 131.06 89.75) (width 0.3) (layer "F.Cu") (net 2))
 (segment (start 128.35 91.85) (end 130.45 89.75) (width 0.3) (layer "F.Cu") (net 2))
 (segment (start 116.77 85.25) (end 116.77 84.95) (width 0.3) (layer "F.Cu") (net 2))
 (segment (start 115.956016 89.75) (end 115.4 89.193984) (width 0.3) (layer "F.Cu") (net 2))
 (via (at 125.2 87.9) (size 0.6) (drill 0.3) (layers "F.Cu" "B.Cu") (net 2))
 (via (at 125.2 85.25) (size 0.6) (drill 0.3) (layers "F.Cu" "B.Cu") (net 2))
 (segment (start 125.2 87.9) (end 125.2 85.25) (width 0.3) (layer "B.Cu") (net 2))
 (segment (start 121.942894 89.25) (end 123.592894 90.9) (width 0.3) (layer "F.Cu") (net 1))
 (segment (start 116.77 89.25) (end 121.942894 89.25) (width 0.3) (layer "F.Cu") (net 1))
 (segment (start 123.592894 90.9) (end 125.2 90.9) (width 0.3) (layer "F.Cu") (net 1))
 (segment (start 132.06 87.75) (end 131.06 87.75) (width 0.3) (layer "F.Cu") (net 7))
 (segment (start 123.3 89.9) (end 122.15 88.75) (width 0.3) (layer "F.Cu") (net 7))
 (segment (start 122.15 88.75) (end 116.77 88.75) (width 0.3) (layer "F.Cu") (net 7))
 (segment (start 128.005456 87.75) (end 125.855456 89.9) (width 0.3) (layer "F.Cu") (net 7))
 (segment (start 132.06 86.75) (end 132.3 86.99) (width 0.3) (layer "F.Cu") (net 7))
 (segment (start 132.3 87.51) (end 132.06 87.75) (width 0.3) (layer "F.Cu") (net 7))
 (segment (start 125.855456 89.9) (end 123.3 89.9) (width 0.3) (layer "F.Cu") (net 7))
 (segment (start 131.06 87.75) (end 128.005456 87.75) (width 0.3) (layer "F.Cu") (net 7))
 (segment (start 131.06 86.75) (end 132.06 86.75) (width 0.3) (layer "F.Cu") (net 7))
 (segment (start 132.3 86.99) (end 132.3 87.51) (width 0.3) (layer "F.Cu") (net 7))
 (segment (start 116.77 86.25) (end 122.05 86.25) (width 0.3) (layer "F.Cu") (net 4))
 (segment (start 122.05 86.25) (end 122.5 86.7) (width 0.3) (layer "F.Cu") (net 4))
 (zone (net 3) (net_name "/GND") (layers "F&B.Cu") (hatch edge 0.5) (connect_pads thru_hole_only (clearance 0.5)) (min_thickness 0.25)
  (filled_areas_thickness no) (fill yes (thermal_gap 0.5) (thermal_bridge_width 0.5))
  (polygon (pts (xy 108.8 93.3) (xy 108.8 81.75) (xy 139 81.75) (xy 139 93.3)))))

